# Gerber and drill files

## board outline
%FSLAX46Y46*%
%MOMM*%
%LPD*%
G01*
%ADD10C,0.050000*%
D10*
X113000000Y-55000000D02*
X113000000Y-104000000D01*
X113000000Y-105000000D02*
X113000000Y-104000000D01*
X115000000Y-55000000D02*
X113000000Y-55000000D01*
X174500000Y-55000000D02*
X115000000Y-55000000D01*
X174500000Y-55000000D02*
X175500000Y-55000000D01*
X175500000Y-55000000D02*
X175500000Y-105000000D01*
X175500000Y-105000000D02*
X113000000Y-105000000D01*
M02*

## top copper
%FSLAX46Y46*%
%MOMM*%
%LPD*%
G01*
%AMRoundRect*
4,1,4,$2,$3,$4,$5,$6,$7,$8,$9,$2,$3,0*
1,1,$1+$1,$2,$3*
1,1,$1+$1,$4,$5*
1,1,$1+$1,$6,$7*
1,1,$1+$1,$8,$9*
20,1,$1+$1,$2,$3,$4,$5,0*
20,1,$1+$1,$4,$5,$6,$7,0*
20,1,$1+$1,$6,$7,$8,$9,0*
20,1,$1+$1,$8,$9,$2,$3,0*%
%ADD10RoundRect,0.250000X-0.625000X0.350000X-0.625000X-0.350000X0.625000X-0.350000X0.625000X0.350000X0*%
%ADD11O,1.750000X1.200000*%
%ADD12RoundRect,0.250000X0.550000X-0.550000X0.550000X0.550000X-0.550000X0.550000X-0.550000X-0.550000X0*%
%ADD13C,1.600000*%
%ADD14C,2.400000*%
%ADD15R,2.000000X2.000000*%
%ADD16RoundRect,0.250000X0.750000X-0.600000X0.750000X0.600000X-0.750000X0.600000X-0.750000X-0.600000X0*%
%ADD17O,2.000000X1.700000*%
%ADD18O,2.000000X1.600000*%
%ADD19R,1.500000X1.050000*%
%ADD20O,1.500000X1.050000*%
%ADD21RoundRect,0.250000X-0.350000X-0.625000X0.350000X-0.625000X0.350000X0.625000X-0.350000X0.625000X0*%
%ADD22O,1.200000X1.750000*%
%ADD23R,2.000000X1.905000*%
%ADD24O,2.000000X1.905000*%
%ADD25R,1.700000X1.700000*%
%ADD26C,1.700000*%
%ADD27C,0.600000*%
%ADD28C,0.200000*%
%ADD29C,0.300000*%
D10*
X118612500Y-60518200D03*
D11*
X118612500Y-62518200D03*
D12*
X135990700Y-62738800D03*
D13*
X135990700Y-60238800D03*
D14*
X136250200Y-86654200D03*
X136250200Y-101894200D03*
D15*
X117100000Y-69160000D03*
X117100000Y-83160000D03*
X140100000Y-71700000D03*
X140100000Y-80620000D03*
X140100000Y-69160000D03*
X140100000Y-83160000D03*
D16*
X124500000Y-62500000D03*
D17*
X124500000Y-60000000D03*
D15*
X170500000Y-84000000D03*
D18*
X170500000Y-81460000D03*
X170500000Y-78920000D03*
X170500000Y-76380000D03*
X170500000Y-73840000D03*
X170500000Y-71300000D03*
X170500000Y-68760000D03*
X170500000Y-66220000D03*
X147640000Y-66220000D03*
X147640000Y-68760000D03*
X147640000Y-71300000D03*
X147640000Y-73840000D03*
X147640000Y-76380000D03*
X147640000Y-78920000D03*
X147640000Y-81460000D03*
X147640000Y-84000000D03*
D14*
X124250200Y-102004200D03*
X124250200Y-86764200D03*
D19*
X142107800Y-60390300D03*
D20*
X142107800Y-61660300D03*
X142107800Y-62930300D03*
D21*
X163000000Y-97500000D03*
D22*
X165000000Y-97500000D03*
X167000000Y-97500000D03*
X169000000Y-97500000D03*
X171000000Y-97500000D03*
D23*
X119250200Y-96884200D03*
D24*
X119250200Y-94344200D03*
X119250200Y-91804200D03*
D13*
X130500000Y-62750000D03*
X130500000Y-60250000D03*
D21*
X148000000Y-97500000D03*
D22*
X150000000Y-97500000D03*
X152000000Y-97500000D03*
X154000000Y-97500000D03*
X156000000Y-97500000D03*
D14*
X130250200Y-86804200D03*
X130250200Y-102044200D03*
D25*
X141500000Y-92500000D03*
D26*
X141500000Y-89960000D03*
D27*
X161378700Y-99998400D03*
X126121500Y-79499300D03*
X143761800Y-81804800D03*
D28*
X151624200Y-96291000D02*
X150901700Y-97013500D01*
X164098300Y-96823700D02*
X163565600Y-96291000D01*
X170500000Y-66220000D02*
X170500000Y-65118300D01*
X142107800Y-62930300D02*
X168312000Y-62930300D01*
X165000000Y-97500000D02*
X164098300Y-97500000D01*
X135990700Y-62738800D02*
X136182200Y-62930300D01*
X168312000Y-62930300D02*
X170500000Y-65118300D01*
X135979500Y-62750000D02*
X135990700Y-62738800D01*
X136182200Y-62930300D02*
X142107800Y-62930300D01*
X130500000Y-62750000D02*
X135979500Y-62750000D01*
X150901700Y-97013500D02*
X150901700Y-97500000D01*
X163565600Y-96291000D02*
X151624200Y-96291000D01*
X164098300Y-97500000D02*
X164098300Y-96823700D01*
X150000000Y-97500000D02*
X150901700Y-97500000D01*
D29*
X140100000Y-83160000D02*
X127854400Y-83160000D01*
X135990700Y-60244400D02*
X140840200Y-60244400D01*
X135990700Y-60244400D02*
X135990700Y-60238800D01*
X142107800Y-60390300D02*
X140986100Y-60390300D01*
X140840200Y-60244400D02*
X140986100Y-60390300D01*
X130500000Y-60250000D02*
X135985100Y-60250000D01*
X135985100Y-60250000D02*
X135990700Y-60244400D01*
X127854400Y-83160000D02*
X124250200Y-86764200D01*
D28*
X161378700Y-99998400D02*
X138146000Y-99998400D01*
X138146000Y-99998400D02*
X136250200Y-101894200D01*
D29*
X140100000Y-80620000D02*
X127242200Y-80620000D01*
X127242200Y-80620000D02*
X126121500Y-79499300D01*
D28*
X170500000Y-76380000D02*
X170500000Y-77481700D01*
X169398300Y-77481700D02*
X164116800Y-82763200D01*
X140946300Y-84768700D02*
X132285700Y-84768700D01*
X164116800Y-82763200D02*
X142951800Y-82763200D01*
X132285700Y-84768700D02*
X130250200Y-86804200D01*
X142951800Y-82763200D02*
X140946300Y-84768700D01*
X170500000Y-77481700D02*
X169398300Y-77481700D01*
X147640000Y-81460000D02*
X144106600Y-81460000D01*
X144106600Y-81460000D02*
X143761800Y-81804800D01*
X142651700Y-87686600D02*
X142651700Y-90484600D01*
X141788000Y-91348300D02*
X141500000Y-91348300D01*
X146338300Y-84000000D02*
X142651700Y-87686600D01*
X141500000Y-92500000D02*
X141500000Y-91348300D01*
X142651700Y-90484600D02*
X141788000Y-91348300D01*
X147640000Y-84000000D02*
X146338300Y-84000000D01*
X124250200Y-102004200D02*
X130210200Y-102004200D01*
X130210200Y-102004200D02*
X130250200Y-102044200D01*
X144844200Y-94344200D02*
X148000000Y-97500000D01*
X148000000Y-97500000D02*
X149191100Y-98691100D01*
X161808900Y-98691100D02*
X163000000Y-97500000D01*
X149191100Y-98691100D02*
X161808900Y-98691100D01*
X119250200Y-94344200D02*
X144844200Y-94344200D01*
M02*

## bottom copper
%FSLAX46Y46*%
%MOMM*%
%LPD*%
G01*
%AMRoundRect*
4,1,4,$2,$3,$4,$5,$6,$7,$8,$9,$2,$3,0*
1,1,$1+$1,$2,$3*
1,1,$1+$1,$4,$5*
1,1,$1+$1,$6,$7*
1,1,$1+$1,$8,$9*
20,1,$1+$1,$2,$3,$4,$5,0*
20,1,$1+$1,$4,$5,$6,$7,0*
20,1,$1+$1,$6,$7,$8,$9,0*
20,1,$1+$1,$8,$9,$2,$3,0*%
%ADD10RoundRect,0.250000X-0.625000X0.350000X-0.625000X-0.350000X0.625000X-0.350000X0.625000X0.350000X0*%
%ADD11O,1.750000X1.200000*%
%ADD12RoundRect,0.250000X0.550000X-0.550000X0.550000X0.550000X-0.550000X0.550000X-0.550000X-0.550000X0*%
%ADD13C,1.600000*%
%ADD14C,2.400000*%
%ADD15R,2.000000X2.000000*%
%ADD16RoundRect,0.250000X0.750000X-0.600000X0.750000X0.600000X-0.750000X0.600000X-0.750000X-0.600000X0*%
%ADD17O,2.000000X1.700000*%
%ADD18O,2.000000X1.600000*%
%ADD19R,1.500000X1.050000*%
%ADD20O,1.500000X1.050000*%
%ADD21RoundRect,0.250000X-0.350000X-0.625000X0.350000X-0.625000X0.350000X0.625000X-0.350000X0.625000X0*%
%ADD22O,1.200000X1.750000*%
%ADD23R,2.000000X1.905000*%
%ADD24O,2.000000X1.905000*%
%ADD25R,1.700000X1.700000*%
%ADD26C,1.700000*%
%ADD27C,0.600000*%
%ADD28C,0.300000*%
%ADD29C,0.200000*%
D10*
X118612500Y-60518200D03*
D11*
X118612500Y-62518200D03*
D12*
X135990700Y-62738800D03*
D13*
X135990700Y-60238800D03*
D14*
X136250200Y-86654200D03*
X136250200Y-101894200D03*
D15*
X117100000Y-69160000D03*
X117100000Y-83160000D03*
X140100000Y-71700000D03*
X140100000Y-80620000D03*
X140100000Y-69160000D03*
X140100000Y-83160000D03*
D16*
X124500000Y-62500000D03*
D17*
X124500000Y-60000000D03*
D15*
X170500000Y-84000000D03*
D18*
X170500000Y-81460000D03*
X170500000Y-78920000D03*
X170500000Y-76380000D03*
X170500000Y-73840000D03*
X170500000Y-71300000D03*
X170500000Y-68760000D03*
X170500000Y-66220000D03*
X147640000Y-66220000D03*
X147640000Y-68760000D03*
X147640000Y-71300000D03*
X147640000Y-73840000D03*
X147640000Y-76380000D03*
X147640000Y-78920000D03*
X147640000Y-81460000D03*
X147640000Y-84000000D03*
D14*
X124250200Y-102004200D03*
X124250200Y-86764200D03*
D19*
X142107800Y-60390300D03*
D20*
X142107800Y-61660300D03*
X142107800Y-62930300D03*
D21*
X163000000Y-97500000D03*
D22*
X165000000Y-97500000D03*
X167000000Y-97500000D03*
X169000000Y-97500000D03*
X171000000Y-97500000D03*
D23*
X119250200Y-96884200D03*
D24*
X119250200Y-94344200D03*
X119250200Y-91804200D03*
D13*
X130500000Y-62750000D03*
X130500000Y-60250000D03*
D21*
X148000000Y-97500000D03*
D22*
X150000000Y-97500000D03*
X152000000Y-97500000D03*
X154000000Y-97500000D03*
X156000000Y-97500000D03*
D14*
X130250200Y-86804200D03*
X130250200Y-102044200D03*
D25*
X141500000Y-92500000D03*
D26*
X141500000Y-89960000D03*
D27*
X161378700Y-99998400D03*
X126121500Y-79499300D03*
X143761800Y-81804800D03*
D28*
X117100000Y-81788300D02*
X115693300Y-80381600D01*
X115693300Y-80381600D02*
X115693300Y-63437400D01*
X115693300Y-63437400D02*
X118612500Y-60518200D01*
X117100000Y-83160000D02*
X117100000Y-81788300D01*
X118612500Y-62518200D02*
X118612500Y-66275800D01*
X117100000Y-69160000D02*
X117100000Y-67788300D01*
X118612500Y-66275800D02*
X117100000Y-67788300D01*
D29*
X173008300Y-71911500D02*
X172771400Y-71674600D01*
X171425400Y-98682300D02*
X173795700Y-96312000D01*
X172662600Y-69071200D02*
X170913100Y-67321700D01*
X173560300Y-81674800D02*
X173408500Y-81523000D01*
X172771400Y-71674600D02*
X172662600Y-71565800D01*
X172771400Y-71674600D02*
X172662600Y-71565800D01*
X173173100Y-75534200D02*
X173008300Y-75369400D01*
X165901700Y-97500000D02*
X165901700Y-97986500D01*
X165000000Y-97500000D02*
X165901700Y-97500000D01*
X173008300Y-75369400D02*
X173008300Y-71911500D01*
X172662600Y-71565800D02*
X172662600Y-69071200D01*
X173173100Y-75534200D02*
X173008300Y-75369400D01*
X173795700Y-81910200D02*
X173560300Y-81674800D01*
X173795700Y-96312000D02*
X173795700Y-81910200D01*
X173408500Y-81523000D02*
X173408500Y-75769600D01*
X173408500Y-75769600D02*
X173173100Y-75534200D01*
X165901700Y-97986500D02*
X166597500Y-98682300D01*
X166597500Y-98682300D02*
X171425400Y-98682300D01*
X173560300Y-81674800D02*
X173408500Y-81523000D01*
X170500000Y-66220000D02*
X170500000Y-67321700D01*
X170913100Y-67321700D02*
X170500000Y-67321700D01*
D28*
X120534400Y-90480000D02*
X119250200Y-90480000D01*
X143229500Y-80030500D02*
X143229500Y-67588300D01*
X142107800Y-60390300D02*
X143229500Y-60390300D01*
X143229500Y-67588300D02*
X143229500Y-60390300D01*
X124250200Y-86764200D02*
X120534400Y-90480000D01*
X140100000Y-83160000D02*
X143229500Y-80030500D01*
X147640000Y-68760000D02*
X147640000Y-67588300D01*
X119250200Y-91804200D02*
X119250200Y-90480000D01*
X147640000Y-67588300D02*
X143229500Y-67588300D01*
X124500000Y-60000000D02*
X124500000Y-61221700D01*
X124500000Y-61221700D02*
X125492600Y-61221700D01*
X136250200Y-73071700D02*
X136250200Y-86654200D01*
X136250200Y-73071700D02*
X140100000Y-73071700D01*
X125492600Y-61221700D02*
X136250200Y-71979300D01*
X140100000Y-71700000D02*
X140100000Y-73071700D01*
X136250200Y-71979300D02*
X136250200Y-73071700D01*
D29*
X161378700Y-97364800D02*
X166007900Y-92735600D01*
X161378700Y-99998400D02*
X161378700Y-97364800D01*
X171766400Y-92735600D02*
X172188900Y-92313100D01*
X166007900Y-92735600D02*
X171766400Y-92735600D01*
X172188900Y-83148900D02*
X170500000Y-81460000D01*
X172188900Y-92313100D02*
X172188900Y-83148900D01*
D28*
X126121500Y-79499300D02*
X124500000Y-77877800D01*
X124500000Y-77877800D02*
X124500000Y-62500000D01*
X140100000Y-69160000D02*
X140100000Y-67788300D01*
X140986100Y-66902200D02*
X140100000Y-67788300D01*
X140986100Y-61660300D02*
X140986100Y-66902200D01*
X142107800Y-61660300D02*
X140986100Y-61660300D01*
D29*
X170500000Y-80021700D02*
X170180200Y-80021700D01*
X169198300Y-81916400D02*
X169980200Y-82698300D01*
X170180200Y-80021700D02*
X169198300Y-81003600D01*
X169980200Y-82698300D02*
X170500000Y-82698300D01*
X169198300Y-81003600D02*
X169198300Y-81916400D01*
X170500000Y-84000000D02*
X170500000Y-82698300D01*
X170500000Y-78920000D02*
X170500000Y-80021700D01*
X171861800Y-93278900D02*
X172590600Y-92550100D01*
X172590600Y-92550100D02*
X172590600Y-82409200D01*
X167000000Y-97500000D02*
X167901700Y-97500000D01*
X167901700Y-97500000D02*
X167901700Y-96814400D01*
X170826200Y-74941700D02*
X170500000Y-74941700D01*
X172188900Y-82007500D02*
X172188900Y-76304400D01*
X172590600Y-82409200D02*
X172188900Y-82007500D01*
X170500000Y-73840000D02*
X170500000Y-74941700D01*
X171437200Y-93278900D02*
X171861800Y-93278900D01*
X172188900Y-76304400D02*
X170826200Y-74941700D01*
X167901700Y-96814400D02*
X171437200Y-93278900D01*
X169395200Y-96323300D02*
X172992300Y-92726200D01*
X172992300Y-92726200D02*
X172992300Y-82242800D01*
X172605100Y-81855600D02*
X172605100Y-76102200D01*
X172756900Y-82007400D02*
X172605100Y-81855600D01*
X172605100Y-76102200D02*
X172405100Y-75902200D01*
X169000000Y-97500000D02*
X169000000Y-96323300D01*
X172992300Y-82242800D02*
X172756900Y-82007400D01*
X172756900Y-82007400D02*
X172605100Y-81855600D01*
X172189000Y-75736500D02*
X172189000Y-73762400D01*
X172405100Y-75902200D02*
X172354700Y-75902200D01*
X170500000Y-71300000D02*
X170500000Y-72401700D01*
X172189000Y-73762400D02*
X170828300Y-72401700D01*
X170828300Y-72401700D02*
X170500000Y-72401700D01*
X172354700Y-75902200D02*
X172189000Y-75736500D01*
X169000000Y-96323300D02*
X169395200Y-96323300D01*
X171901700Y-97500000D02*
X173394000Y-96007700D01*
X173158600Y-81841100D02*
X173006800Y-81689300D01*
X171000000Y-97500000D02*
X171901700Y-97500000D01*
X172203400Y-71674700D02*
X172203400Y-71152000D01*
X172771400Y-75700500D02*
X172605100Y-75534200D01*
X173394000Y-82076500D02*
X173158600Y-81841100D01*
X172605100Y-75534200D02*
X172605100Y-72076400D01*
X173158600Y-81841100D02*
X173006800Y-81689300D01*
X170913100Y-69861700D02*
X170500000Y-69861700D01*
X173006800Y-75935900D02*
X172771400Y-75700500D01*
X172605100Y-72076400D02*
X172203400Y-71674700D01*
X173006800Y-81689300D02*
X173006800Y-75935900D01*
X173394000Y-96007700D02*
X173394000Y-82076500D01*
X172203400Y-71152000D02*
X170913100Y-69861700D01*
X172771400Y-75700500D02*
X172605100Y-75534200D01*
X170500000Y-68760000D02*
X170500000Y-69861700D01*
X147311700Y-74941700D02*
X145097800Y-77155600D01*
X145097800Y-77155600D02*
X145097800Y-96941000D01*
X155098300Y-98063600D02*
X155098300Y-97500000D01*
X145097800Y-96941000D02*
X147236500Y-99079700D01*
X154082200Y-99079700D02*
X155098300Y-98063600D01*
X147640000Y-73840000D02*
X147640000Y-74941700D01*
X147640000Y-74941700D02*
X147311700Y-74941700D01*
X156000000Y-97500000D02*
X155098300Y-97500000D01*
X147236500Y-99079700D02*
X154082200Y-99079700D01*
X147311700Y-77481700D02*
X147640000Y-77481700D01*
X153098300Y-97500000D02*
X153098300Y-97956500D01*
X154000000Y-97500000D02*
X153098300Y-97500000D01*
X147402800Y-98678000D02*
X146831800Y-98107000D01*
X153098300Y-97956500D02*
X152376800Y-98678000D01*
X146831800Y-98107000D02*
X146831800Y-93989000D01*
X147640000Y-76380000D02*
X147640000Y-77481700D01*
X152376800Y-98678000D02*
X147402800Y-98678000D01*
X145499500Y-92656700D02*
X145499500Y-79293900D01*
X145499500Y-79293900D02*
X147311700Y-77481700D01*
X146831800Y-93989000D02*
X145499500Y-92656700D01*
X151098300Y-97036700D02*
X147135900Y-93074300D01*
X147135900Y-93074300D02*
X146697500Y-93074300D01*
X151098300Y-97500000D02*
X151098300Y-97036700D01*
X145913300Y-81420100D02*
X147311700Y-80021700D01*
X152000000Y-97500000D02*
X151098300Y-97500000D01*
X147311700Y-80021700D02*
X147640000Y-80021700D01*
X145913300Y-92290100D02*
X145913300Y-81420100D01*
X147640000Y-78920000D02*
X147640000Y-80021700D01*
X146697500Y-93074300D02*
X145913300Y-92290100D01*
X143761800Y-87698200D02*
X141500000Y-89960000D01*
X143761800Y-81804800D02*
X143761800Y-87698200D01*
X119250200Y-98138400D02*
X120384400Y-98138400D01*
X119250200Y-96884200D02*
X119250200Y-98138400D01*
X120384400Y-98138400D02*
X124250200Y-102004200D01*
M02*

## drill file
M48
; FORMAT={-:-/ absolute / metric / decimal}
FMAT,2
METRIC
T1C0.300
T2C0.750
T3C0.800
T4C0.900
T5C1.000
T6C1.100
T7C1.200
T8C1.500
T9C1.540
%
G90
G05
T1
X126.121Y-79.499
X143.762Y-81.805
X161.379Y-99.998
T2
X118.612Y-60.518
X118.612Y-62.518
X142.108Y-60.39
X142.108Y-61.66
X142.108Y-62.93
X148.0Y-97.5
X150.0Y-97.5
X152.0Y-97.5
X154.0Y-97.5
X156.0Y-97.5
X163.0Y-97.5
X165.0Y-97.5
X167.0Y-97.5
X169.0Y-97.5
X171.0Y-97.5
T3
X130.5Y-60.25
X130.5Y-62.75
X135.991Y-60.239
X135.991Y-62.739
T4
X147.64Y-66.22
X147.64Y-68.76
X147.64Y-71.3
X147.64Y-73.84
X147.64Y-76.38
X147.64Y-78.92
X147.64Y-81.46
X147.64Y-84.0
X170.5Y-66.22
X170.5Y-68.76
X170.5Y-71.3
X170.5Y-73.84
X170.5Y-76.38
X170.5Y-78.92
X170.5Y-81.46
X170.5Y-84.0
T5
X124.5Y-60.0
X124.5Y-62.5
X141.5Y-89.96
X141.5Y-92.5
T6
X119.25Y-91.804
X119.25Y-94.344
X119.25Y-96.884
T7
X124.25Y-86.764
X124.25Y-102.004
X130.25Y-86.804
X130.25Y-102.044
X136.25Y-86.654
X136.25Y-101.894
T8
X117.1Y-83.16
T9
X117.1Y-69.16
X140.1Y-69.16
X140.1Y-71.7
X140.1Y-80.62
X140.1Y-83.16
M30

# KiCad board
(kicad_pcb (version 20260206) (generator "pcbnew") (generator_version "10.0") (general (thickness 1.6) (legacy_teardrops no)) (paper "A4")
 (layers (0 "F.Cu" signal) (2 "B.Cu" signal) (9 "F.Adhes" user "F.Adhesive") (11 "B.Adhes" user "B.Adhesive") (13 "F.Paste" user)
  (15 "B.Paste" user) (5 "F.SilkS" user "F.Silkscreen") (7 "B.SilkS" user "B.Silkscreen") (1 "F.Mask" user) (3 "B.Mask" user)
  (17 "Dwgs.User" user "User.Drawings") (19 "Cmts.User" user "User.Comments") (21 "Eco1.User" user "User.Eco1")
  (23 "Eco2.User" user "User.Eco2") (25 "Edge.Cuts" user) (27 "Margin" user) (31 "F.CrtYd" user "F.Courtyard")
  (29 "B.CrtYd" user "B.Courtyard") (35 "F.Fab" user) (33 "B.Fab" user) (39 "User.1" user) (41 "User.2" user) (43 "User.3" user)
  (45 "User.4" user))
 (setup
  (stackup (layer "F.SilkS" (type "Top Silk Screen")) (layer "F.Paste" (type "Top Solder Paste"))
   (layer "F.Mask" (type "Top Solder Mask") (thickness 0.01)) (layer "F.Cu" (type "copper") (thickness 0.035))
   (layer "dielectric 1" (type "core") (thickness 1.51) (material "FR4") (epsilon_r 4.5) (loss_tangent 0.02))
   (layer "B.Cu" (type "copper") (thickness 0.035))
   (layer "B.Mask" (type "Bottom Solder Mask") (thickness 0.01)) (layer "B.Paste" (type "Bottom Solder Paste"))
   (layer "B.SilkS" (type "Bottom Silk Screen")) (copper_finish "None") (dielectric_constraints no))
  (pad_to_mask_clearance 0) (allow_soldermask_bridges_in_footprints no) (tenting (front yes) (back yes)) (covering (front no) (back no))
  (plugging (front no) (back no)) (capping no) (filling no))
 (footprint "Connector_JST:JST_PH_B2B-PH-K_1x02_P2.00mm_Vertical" (layer "F.Cu") (at 118.6125 60.5182 -90)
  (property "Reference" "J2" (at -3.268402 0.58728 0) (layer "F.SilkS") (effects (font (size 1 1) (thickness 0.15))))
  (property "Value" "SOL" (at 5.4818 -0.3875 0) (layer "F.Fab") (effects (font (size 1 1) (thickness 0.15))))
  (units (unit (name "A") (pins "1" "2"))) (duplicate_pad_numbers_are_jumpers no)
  (pad "1" thru_hole roundrect (at 0 0 270) (size 1.2 1.75) (drill 0.75) (layers "*.Cu" "*.Mask") (remove_unused_layers no)
   (roundrect_rratio 0.208333) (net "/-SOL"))
  (pad "2" thru_hole oval (at 2 0 270) (size 1.2 1.75) (drill 0.75) (layers "*.Cu" "*.Mask") (remove_unused_layers no) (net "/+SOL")))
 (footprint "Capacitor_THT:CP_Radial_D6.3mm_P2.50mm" (layer "F.Cu") (at 135.9907 62.7388 90)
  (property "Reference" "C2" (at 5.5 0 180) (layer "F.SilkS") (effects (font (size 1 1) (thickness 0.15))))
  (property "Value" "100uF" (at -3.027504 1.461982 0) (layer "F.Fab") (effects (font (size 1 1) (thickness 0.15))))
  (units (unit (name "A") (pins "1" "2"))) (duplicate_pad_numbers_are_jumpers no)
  (pad "1" thru_hole roundrect (at 0 0 90) (size 1.6 1.6) (drill 0.8) (layers "*.Cu" "*.Mask") (remove_unused_layers no)
   (roundrect_rratio 0.15625) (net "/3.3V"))
  (pad "2" thru_hole circle (at 2.5 0 90) (size 1.6 1.6) (drill 0.8) (layers "*.Cu" "*.Mask") (remove_unused_layers no) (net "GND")))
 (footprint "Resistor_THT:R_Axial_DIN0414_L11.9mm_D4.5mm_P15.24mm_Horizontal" (layer "F.Cu") (at 136.2502 86.6542 -90)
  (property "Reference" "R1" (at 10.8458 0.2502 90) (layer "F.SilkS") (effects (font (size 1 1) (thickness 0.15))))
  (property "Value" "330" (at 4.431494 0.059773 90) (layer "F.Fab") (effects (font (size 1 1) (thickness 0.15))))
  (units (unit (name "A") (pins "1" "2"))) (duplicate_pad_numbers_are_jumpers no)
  (pad "1" thru_hole circle (at 0 0 270) (size 2.4 2.4) (drill 1.2) (layers "*.Cu" "*.Mask") (remove_unused_layers no) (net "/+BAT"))
  (pad "2" thru_hole circle (at 15.24 0 270) (size 2.4 2.4) (drill 1.2) (layers "*.Cu" "*.Mask") (remove_unused_layers no)
   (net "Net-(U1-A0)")))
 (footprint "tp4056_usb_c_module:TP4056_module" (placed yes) (layer "F.Cu") (at 115.5 67.5)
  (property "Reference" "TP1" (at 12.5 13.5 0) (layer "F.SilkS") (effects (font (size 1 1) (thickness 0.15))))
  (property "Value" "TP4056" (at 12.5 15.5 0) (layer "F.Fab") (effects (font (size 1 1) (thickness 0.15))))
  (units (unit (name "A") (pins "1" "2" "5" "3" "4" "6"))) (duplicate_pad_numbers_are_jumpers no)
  (pad "1" thru_hole rect (at 1.6 1.66) (size 2 2) (drill 1.54) (layers "*.Cu" "*.Mask") (remove_unused_layers no) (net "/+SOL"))
  (pad "2" thru_hole rect (at 1.6 15.66) (size 2 2) (drill 1.5) (layers "*.Cu" "*.Mask") (remove_unused_layers no) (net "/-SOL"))
  (pad "3" thru_hole rect (at 24.6 4.2) (size 2 2) (drill 1.54) (layers "*.Cu" "*.Mask") (remove_unused_layers no) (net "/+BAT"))
  (pad "4" thru_hole rect (at 24.6 13.12) (size 2 2) (drill 1.54) (layers "*.Cu" "*.Mask") (remove_unused_layers no) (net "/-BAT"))
  (pad "5" thru_hole rect (at 24.6 1.66) (size 2 2) (drill 1.54) (layers "*.Cu" "*.Mask") (remove_unused_layers no) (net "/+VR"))
  (pad "6" thru_hole rect (at 24.6 15.66) (size 2 2) (drill 1.54) (layers "*.Cu" "*.Mask") (remove_unused_layers no) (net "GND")))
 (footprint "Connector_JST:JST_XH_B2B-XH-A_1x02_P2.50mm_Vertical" (layer "F.Cu") (at 124.5 62.5 90)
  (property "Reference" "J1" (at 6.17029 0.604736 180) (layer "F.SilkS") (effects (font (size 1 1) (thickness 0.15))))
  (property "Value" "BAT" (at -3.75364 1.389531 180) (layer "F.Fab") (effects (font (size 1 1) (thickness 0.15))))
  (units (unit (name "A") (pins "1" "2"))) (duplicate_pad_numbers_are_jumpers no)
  (pad "1" thru_hole roundrect (at 0 0 90) (size 1.7 2) (drill 1) (layers "*.Cu" "*.Mask") (remove_unused_layers no)
   (roundrect_rratio 0.147059) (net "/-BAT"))
  (pad "2" thru_hole oval (at 2.5 0 90) (size 1.7 2) (drill 1) (layers "*.Cu" "*.Mask") (remove_unused_layers no) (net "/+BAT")))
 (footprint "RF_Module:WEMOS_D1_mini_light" (layer "F.Cu") (at 170.5 84 180)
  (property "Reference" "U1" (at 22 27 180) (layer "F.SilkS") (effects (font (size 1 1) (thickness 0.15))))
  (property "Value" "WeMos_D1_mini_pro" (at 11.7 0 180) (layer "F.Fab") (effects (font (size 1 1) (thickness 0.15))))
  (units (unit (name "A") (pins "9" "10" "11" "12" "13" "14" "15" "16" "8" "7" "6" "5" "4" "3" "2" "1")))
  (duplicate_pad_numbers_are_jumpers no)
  (pad "1" thru_hole rect (at 0 0 180) (size 2 2) (drill 0.9) (layers "*.Cu" "*.Mask") (remove_unused_layers no) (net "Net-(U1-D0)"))
  (pad "2" thru_hole oval (at 0 2.54 180) (size 2 1.6) (drill 0.9) (layers "*.Cu" "*.Mask") (remove_unused_layers no) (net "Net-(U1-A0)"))
  (pad "3" thru_hole oval (at 0 5.08 180) (size 2 1.6) (drill 0.9) (layers "*.Cu" "*.Mask") (remove_unused_layers no) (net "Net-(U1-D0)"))
  (pad "4" thru_hole oval (at 0 7.62 180) (size 2 1.6) (drill 0.9) (layers "*.Cu" "*.Mask") (remove_unused_layers no) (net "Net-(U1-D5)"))
  (pad "5" thru_hole oval (at 0 10.16 180) (size 2 1.6) (drill 0.9) (layers "*.Cu" "*.Mask") (remove_unused_layers no) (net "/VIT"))
  (pad "6" thru_hole oval (at 0 12.7 180) (size 2 1.6) (drill 0.9) (layers "*.Cu" "*.Mask") (remove_unused_layers no) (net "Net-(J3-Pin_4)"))
  (pad "7" thru_hole oval (at 0 15.24 180) (size 2 1.6) (drill 0.9) (layers "*.Cu" "*.Mask") (remove_unused_layers no)
   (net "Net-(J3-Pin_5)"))
  (pad "8" thru_hole oval (at 0 17.78 180) (size 2 1.6) (drill 0.9) (layers "*.Cu" "*.Mask") (remove_unused_layers no) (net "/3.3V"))
  (pad "9" thru_hole oval (at 22.86 17.78 180) (size 2 1.6) (drill 0.9) (layers "*.Cu" "*.Mask") (remove_unused_layers no)
   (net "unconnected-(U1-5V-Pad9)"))
  (pad "10" thru_hole oval (at 22.86 15.24 180) (size 2 1.6) (drill 0.9) (layers "*.Cu" "*.Mask") (remove_unused_layers no) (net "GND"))
  (pad "11" thru_hole oval (at 22.86 12.7 180) (size 2 1.6) (drill 0.9) (layers "*.Cu" "*.Mask") (remove_unused_layers no)
   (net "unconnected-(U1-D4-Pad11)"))
  (pad "12" thru_hole oval (at 22.86 10.16 180) (size 2 1.6) (drill 0.9) (layers "*.Cu" "*.Mask") (remove_unused_layers no)
   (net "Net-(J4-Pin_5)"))
  (pad "13" thru_hole oval (at 22.86 7.62 180) (size 2 1.6) (drill 0.9) (layers "*.Cu" "*.Mask") (remove_unused_layers no)
   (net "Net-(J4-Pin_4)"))
  (pad "14" thru_hole oval (at 22.86 5.08 180) (size 2 1.6) (drill 0.9) (layers "*.Cu" "*.Mask") (remove_unused_layers no)
   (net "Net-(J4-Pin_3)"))
  (pad "15" thru_hole oval (at 22.86 2.54 180) (size 2 1.6) (drill 0.9) (layers "*.Cu" "*.Mask") (remove_unused_layers no) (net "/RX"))
  (pad "16" thru_hole oval (at 22.86 0 180) (size 2 1.6) (drill 0.9) (layers "*.Cu" "*.Mask") (remove_unused_layers no) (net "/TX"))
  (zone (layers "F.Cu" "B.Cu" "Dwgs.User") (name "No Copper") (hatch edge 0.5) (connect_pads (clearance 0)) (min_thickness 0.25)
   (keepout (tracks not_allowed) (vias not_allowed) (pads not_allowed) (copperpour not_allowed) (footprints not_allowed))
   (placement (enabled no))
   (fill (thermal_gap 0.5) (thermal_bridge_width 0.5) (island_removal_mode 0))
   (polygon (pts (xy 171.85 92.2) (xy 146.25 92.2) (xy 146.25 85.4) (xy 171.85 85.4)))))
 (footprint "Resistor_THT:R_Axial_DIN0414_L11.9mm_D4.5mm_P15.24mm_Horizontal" (layer "F.Cu") (at 124.2502 102.0042 90)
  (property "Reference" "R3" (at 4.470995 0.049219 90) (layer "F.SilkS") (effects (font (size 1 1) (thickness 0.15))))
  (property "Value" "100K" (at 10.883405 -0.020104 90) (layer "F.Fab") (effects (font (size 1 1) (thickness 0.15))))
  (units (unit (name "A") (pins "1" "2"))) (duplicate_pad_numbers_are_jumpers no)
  (pad "1" thru_hole circle (at 0 0 90) (size 2.4 2.4) (drill 1.2) (layers "*.Cu" "*.Mask") (remove_unused_layers no) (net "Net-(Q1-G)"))
  (pad "2" thru_hole circle (at 15.24 0 90) (size 2.4 2.4) (drill 1.2) (layers "*.Cu" "*.Mask") (remove_unused_layers no) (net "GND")))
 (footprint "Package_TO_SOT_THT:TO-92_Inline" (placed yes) (layer "F.Cu") (at 142.1078 60.3903 -90)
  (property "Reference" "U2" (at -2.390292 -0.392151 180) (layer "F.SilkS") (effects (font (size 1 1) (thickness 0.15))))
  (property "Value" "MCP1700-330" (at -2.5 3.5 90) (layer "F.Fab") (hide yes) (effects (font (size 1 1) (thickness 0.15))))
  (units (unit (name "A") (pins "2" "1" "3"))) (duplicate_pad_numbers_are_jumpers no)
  (pad "1" thru_hole rect (at 0 0 270) (size 1.05 1.5) (drill 0.75) (layers "*.Cu" "*.Mask") (remove_unused_layers no) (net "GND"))
  (pad "2" thru_hole oval (at 1.27 0 270) (size 1.05 1.5) (drill 0.75) (layers "*.Cu" "*.Mask") (remove_unused_layers no) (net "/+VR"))
  (pad "3" thru_hole oval (at 2.54 0 270) (size 1.05 1.5) (drill 0.75) (layers "*.Cu" "*.Mask") (remove_unused_layers no) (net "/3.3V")))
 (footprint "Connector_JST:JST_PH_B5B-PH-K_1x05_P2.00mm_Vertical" (layer "F.Cu") (at 163 97.5)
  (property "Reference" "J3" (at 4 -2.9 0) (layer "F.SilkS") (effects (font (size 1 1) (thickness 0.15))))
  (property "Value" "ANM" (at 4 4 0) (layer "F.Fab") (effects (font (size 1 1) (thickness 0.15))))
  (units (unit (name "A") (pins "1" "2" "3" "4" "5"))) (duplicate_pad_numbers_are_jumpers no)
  (pad "1" thru_hole roundrect (at 0 0) (size 1.2 1.75) (drill 0.75) (layers "*.Cu" "*.Mask") (remove_unused_layers no)
   (roundrect_rratio 0.208333) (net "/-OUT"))
  (pad "2" thru_hole oval (at 2 0) (size 1.2 1.75) (drill 0.75) (layers "*.Cu" "*.Mask") (remove_unused_layers no) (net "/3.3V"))
  (pad "3" thru_hole oval (at 4 0) (size 1.2 1.75) (drill 0.75) (layers "*.Cu" "*.Mask") (remove_unused_layers no) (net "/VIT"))
  (pad "4" thru_hole oval (at 6 0) (size 1.2 1.75) (drill 0.75) (layers "*.Cu" "*.Mask") (remove_unused_layers no) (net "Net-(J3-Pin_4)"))
  (pad "5" thru_hole oval (at 8 0) (size 1.2 1.75) (drill 0.75) (layers "*.Cu" "*.Mask") (remove_unused_layers no) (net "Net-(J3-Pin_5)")))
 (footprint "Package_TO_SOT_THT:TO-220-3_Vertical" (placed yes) (layer "F.Cu") (at 119.2502 96.8842 90)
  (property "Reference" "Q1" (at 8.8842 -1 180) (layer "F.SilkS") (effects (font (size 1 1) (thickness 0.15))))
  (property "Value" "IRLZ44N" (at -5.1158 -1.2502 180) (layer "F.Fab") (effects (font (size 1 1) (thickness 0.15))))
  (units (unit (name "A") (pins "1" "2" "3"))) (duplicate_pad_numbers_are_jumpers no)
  (pad "1" thru_hole rect (at 0 0 90) (size 1.905 2) (drill 1.1) (layers "*.Cu" "*.Mask") (remove_unused_layers no) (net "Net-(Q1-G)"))
  (pad "2" thru_hole oval (at 2.54 0 90) (size 1.905 2) (drill 1.1) (layers "*.Cu" "*.Mask") (remove_unused_layers no) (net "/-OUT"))
  (pad "3" thru_hole oval (at 5.08 0 90) (size 1.905 2) (drill 1.1) (layers "*.Cu" "*.Mask") (remove_unused_layers no) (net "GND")))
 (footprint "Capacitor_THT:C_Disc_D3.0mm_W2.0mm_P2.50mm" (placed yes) (layer "F.Cu") (at 130.5 62.75 90)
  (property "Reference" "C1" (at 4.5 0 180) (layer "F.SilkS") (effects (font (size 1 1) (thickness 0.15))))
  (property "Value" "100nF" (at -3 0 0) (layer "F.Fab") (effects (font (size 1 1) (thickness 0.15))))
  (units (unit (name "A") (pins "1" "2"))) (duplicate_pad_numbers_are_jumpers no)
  (pad "1" thru_hole circle (at 0 0 90) (size 1.6 1.6) (drill 0.8) (layers "*.Cu" "*.Mask") (remove_unused_layers no) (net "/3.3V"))
  (pad "2" thru_hole circle (at 2.5 0 90) (size 1.6 1.6) (drill 0.8) (layers "*.Cu" "*.Mask") (remove_unused_layers no) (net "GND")))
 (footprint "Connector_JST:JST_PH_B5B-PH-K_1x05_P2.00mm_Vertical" (layer "F.Cu") (at 148 97.5)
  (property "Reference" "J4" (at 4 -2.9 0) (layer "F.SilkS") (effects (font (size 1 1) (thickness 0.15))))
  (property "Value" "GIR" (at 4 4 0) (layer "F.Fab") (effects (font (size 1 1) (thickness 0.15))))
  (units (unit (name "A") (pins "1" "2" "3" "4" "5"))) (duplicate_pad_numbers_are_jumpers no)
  (pad "1" thru_hole roundrect (at 0 0) (size 1.2 1.75) (drill 0.75) (layers "*.Cu" "*.Mask") (remove_unused_layers no)
   (roundrect_rratio 0.208333) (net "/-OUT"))
  (pad "2" thru_hole oval (at 2 0) (size 1.2 1.75) (drill 0.75) (layers "*.Cu" "*.Mask") (remove_unused_layers no) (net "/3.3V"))
  (pad "3" thru_hole oval (at 4 0) (size 1.2 1.75) (drill 0.75) (layers "*.Cu" "*.Mask") (remove_unused_layers no) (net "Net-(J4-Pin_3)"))
  (pad "4" thru_hole oval (at 6 0) (size 1.2 1.75) (drill 0.75) (layers "*.Cu" "*.Mask") (remove_unused_layers no) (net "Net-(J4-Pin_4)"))
  (pad "5" thru_hole oval (at 8 0) (size 1.2 1.75) (drill 0.75) (layers "*.Cu" "*.Mask") (remove_unused_layers no) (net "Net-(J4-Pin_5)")))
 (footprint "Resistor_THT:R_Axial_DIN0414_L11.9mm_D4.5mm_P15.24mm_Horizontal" (layer "F.Cu") (at 130.2502 86.8042 -90)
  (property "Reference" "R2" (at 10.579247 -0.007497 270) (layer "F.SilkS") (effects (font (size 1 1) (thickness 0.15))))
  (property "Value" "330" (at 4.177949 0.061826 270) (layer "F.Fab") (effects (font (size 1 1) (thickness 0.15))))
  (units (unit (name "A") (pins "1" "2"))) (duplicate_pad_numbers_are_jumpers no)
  (pad "1" thru_hole circle (at 0 0 270) (size 2.4 2.4) (drill 1.2) (layers "*.Cu" "*.Mask") (remove_unused_layers no) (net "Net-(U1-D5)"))
  (pad "2" thru_hole circle (at 15.24 0 270) (size 2.4 2.4) (drill 1.2) (layers "*.Cu" "*.Mask") (remove_unused_layers no)
   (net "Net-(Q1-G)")))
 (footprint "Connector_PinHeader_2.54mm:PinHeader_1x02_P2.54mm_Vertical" (layer "F.Cu") (at 141.5 92.5 180)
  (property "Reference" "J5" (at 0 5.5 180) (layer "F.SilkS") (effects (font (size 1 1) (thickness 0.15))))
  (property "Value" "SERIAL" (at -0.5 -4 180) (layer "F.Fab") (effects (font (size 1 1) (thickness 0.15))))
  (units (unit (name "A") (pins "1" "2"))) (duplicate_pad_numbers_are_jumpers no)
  (pad "1" thru_hole rect (at 0 0 180) (size 1.7 1.7) (drill 1) (layers "*.Cu" "*.Mask") (remove_unused_layers no) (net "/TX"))
  (pad "2" thru_hole circle (at 0 2.54 180) (size 1.7 1.7) (drill 1) (layers "*.Cu" "*.Mask") (remove_unused_layers no) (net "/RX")))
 (gr_line (start 113 55) (end 113 104) (stroke (width 0.05) (type default)) (layer "Edge.Cuts"))
 (gr_line (start 113 105) (end 113 104) (stroke (width 0.05) (type default)) (layer "Edge.Cuts"))
 (gr_line (start 115 55) (end 113 55) (stroke (width 0.05) (type default)) (layer "Edge.Cuts"))
 (gr_line (start 174.5 55) (end 115 55) (stroke (width 0.05) (type default)) (layer "Edge.Cuts"))
 (gr_line (start 174.5 55) (end 175.5 55) (stroke (width 0.05) (type default)) (layer "Edge.Cuts"))
 (gr_line (start 175.5 55) (end 175.5 105) (stroke (width 0.05) (type default)) (layer "Edge.Cuts"))
 (gr_line (start 175.5 105) (end 113 105) (stroke (width 0.05) (type default)) (layer "Edge.Cuts"))
 (segment (start 117.1 81.7883) (end 115.6933 80.3816) (width 0.3) (layer "B.Cu") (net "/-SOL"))
 (segment (start 115.6933 80.3816) (end 115.6933 63.4374) (width 0.3) (layer "B.Cu") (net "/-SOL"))
 (segment (start 115.6933 63.4374) (end 118.6125 60.5182) (width 0.3) (layer "B.Cu") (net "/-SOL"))
 (segment (start 117.1 83.16) (end 117.1 81.7883) (width 0.3) (layer "B.Cu") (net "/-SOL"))
 (segment (start 118.6125 62.5182) (end 118.6125 66.2758) (width 0.3) (layer "B.Cu") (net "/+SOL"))
 (segment (start 117.1 69.16) (end 117.1 67.7883) (width 0.3) (layer "B.Cu") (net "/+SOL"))
 (segment (start 118.6125 66.2758) (end 117.1 67.7883) (width 0.3) (layer "B.Cu") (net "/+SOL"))
 (segment (start 151.6242 96.291) (end 150.9017 97.0135) (width 0.2) (layer "F.Cu") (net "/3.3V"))
 (segment (start 164.0983 96.8237) (end 163.5656 96.291) (width 0.2) (layer "F.Cu") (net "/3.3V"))
 (segment (start 170.5 66.22) (end 170.5 65.1183) (width 0.2) (layer "F.Cu") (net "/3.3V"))
 (segment (start 142.1078 62.9303) (end 168.312 62.9303) (width 0.2) (layer "F.Cu") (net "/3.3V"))
 (segment (start 165 97.5) (end 164.0983 97.5) (width 0.2) (layer "F.Cu") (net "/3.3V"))
 (segment (start 135.9907 62.7388) (end 136.1822 62.9303) (width 0.2) (layer "F.Cu") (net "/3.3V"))
 (segment (start 168.312 62.9303) (end 170.5 65.1183) (width 0.2) (layer "F.Cu") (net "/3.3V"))
 (segment (start 135.9795 62.75) (end 135.9907 62.7388) (width 0.2) (layer "F.Cu") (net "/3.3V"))
 (segment (start 136.1822 62.9303) (end 142.1078 62.9303) (width 0.2) (layer "F.Cu") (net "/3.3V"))
 (segment (start 130.5 62.75) (end 135.9795 62.75) (width 0.2) (layer "F.Cu") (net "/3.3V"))
 (segment (start 150.9017 97.0135) (end 150.9017 97.5) (width 0.2) (layer "F.Cu") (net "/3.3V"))
 (segment (start 163.5656 96.291) (end 151.6242 96.291) (width 0.2) (layer "F.Cu") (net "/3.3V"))
 (segment (start 164.0983 97.5) (end 164.0983 96.8237) (width 0.2) (layer "F.Cu") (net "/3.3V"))
 (segment (start 150 97.5) (end 150.9017 97.5) (width 0.2) (layer "F.Cu") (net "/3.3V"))
 (segment (start 173.0083 71.9115) (end 172.7714 71.6746) (width 0.2) (layer "B.Cu") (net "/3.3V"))
 (segment (start 171.4254 98.6823) (end 173.7957 96.312) (width 0.2) (layer "B.Cu") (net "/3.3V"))
 (segment (start 172.6626 69.0712) (end 170.9131 67.3217) (width 0.2) (layer "B.Cu") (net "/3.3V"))
 (segment (start 173.5603 81.6748) (end 173.4085 81.523) (width 0.2) (layer "B.Cu") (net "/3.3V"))
 (segment (start 172.7714 71.6746) (end 172.6626 71.5658) (width 0.2) (layer "B.Cu") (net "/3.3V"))
 (segment (start 172.7714 71.6746) (end 172.6626 71.5658) (width 0.2) (layer "B.Cu") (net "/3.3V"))
 (segment (start 173.1731 75.5342) (end 173.0083 75.3694) (width 0.2) (layer "B.Cu") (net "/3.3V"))
 (segment (start 165.9017 97.5) (end 165.9017 97.9865) (width 0.2) (layer "B.Cu") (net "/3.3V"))
 (segment (start 165 97.5) (end 165.9017 97.5) (width 0.2) (layer "B.Cu") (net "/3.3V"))
 (segment (start 173.0083 75.3694) (end 173.0083 71.9115) (width 0.2) (layer "B.Cu") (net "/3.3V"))
 (segment (start 172.6626 71.5658) (end 172.6626 69.0712) (width 0.2) (layer "B.Cu") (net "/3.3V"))
 (segment (start 173.1731 75.5342) (end 173.0083 75.3694) (width 0.2) (layer "B.Cu") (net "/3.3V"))
 (segment (start 173.7957 81.9102) (end 173.5603 81.6748) (width 0.2) (layer "B.Cu") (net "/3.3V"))
 (segment (start 173.7957 96.312) (end 173.7957 81.9102) (width 0.2) (layer "B.Cu") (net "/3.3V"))
 (segment (start 173.4085 81.523) (end 173.4085 75.7696) (width 0.2) (layer "B.Cu") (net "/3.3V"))
 (segment (start 173.4085 75.7696) (end 173.1731 75.5342) (width 0.2) (layer "B.Cu") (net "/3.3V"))
 (segment (start 165.9017 97.9865) (end 166.5975 98.6823) (width 0.2) (layer "B.Cu") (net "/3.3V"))
 (segment (start 166.5975 98.6823) (end 171.4254 98.6823) (width 0.2) (layer "B.Cu") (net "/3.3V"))
 (segment (start 173.5603 81.6748) (end 173.4085 81.523) (width 0.2) (layer "B.Cu") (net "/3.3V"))
 (segment (start 170.5 66.22) (end 170.5 67.3217) (width 0.2) (layer "B.Cu") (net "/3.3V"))
 (segment (start 170.9131 67.3217) (end 170.5 67.3217) (width 0.2) (layer "B.Cu") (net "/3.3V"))
 (segment (start 140.1 83.16) (end 127.8544 83.16) (width 0.3) (layer "F.Cu") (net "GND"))
 (segment (start 135.9907 60.2444) (end 140.8402 60.2444) (width 0.3) (layer "F.Cu") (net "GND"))
 (segment (start 135.9907 60.2444) (end 135.9907 60.2388) (width 0.3) (layer "F.Cu") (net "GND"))
 (segment (start 142.1078 60.3903) (end 140.9861 60.3903) (width 0.3) (layer "F.Cu") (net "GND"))
 (segment (start 140.8402 60.2444) (end 140.9861 60.3903) (width 0.3) (layer "F.Cu") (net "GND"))
 (segment (start 130.5 60.25) (end 135.9851 60.25) (width 0.3) (layer "F.Cu") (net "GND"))
 (segment (start 135.9851 60.25) (end 135.9907 60.2444) (width 0.3) (layer "F.Cu") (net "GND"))
 (segment (start 127.8544 83.16) (end 124.2502 86.7642) (width 0.3) (layer "F.Cu") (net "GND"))
 (segment (start 120.5344 90.48) (end 119.2502 90.48) (width 0.3) (layer "B.Cu") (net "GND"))
 (segment (start 143.2295 80.0305) (end 143.2295 67.5883) (width 0.3) (layer "B.Cu") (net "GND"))
 (segment (start 142.1078 60.3903) (end 143.2295 60.3903) (width 0.3) (layer "B.Cu") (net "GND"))
 (segment (start 143.2295 67.5883) (end 143.2295 60.3903) (width 0.3) (layer "B.Cu") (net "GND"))
 (segment (start 124.2502 86.7642) (end 120.5344 90.48) (width 0.3) (layer "B.Cu") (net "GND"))
 (segment (start 140.1 83.16) (end 143.2295 80.0305) (width 0.3) (layer "B.Cu") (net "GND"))
 (segment (start 147.64 68.76) (end 147.64 67.5883) (width 0.3) (layer "B.Cu") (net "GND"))
 (segment (start 119.2502 91.8042) (end 119.2502 90.48) (width 0.3) (layer "B.Cu") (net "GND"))
 (segment (start 147.64 67.5883) (end 143.2295 67.5883) (width 0.3) (layer "B.Cu") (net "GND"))
 (segment (start 124.5 60) (end 124.5 61.2217) (width 0.3) (layer "B.Cu") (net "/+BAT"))
 (segment (start 124.5 61.2217) (end 125.4926 61.2217) (width 0.3) (layer "B.Cu") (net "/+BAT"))
 (segment (start 136.2502 73.0717) (end 136.2502 86.6542) (width 0.3) (layer "B.Cu") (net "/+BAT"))
 (segment (start 136.2502 73.0717) (end 140.1 73.0717) (width 0.3) (layer "B.Cu") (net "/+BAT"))
 (segment (start 125.4926 61.2217) (end 136.2502 71.9793) (width 0.3) (layer "B.Cu") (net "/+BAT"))
 (segment (start 140.1 71.7) (end 140.1 73.0717) (width 0.3) (layer "B.Cu") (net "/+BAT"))
 (segment (start 136.2502 71.9793) (end 136.2502 73.0717) (width 0.3) (layer "B.Cu") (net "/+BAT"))
 (segment (start 161.3787 99.9984) (end 138.146 99.9984) (width 0.2) (layer "F.Cu") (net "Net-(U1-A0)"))
 (segment (start 138.146 99.9984) (end 136.2502 101.8942) (width 0.2) (layer "F.Cu") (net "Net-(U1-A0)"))
 (via (at 161.3787 99.9984) (size 0.6) (drill 0.3) (layers "F.Cu" "B.Cu") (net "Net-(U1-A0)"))
 (segment (start 161.3787 97.3648) (end 166.0079 92.7356) (width 0.2) (layer "B.Cu") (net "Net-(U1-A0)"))
 (segment (start 161.3787 99.9984) (end 161.3787 97.3648) (width 0.2) (layer "B.Cu") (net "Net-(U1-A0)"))
 (segment (start 171.7664 92.7356) (end 172.1889 92.3131) (width 0.2) (layer "B.Cu") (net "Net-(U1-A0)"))
 (segment (start 166.0079 92.7356) (end 171.7664 92.7356) (width 0.2) (layer "B.Cu") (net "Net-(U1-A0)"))
 (segment (start 172.1889 83.1489) (end 170.5 81.46) (width 0.2) (layer "B.Cu") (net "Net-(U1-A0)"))
 (segment (start 172.1889 92.3131) (end 172.1889 83.1489) (width 0.2) (layer "B.Cu") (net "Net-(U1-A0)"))
 (segment (start 140.1 80.62) (end 127.2422 80.62) (width 0.3) (layer "F.Cu") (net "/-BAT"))
 (segment (start 127.2422 80.62) (end 126.1215 79.4993) (width 0.3) (layer "F.Cu") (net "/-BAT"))
 (via (at 126.1215 79.4993) (size 0.6) (drill 0.3) (layers "F.Cu" "B.Cu") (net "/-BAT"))
 (segment (start 126.1215 79.4993) (end 124.5 77.8778) (width 0.3) (layer "B.Cu") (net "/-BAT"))
 (segment (start 124.5 77.8778) (end 124.5 62.5) (width 0.3) (layer "B.Cu") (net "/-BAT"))
 (segment (start 140.1 69.16) (end 140.1 67.7883) (width 0.3) (layer "B.Cu") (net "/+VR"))
 (segment (start 140.9861 66.9022) (end 140.1 67.7883) (width 0.3) (layer "B.Cu") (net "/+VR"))
 (segment (start 140.9861 61.6603) (end 140.9861 66.9022) (width 0.3) (layer "B.Cu") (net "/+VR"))
 (segment (start 142.1078 61.6603) (end 140.9861 61.6603) (width 0.3) (layer "B.Cu") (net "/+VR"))
 (segment (start 170.5 80.0217) (end 170.1802 80.0217) (width 0.2) (layer "B.Cu") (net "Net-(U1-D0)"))
 (segment (start 169.1983 81.9164) (end 169.9802 82.6983) (width 0.2) (layer "B.Cu") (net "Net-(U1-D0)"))
 (segment (start 170.1802 80.0217) (end 169.1983 81.0036) (width 0.2) (layer "B.Cu") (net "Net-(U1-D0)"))
 (segment (start 169.9802 82.6983) (end 170.5 82.6983) (width 0.2) (layer "B.Cu") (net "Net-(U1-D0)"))
 (segment (start 169.1983 81.0036) (end 169.1983 81.9164) (width 0.2) (layer "B.Cu") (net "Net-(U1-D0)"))
 (segment (start 170.5 84) (end 170.5 82.6983) (width 0.2) (layer "B.Cu") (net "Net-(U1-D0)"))
 (segment (start 170.5 78.92) (end 170.5 80.0217) (width 0.2) (layer "B.Cu") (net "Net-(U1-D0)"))
 (segment (start 170.5 76.38) (end 170.5 77.4817) (width 0.2) (layer "F.Cu") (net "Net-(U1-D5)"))
 (segment (start 169.3983 77.4817) (end 164.1168 82.7632) (width 0.2) (layer "F.Cu") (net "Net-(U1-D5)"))
 (segment (start 140.9463 84.7687) (end 132.2857 84.7687) (width 0.2) (layer "F.Cu") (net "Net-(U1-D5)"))
 (segment (start 164.1168 82.7632) (end 142.9518 82.7632) (width 0.2) (layer "F.Cu") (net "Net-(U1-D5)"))
 (segment (start 132.2857 84.7687) (end 130.2502 86.8042) (width 0.2) (layer "F.Cu") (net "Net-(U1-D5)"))
 (segment (start 142.9518 82.7632) (end 140.9463 84.7687) (width 0.2) (layer "F.Cu") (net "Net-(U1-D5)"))
 (segment (start 170.5 77.4817) (end 169.3983 77.4817) (width 0.2) (layer "F.Cu") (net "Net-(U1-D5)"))
 (segment (start 171.8618 93.2789) (end 172.5906 92.5501) (width 0.2) (layer "B.Cu") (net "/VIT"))
 (segment (start 172.5906 92.5501) (end 172.5906 82.4092) (width 0.2) (layer "B.Cu") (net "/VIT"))
 (segment (start 167 97.5) (end 167.9017 97.5) (width 0.2) (layer "B.Cu") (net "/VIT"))
 (segment (start 167.9017 97.5) (end 167.9017 96.8144) (width 0.2) (layer "B.Cu") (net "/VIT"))
 (segment (start 170.8262 74.9417) (end 170.5 74.9417) (width 0.2) (layer "B.Cu") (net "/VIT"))
 (segment (start 172.1889 82.0075) (end 172.1889 76.3044) (width 0.2) (layer "B.Cu") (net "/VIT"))
 (segment (start 172.5906 82.4092) (end 172.1889 82.0075) (width 0.2) (layer "B.Cu") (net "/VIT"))
 (segment (start 170.5 73.84) (end 170.5 74.9417) (width 0.2) (layer "B.Cu") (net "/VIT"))
 (segment (start 171.4372 93.2789) (end 171.8618 93.2789) (width 0.2) (layer "B.Cu") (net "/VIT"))
 (segment (start 172.1889 76.3044) (end 170.8262 74.9417) (width 0.2) (layer "B.Cu") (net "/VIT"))
 (segment (start 167.9017 96.8144) (end 171.4372 93.2789) (width 0.2) (layer "B.Cu") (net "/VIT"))
 (segment (start 169.3952 96.3233) (end 172.9923 92.7262) (width 0.2) (layer "B.Cu") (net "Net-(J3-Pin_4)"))
 (segment (start 172.9923 92.7262) (end 172.9923 82.2428) (width 0.2) (layer "B.Cu") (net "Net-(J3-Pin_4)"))
 (segment (start 172.6051 81.8556) (end 172.6051 76.1022) (width 0.2) (layer "B.Cu") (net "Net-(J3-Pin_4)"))
 (segment (start 172.7569 82.0074) (end 172.6051 81.8556) (width 0.2) (layer "B.Cu") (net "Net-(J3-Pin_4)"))
 (segment (start 172.6051 76.1022) (end 172.4051 75.9022) (width 0.2) (layer "B.Cu") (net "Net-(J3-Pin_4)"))
 (segment (start 169 97.5) (end 169 96.3233) (width 0.2) (layer "B.Cu") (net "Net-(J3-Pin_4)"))
 (segment (start 172.9923 82.2428) (end 172.7569 82.0074) (width 0.2) (layer "B.Cu") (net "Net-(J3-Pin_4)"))
 (segment (start 172.7569 82.0074) (end 172.6051 81.8556) (width 0.2) (layer "B.Cu") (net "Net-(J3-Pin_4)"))
 (segment (start 172.189 75.7365) (end 172.189 73.7624) (width 0.2) (layer "B.Cu") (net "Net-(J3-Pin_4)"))
 (segment (start 172.4051 75.9022) (end 172.3547 75.9022) (width 0.2) (layer "B.Cu") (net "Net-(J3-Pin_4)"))
 (segment (start 170.5 71.3) (end 170.5 72.4017) (width 0.2) (layer "B.Cu") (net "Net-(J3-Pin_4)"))
 (segment (start 172.189 73.7624) (end 170.8283 72.4017) (width 0.2) (layer "B.Cu") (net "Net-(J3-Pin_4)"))
 (segment (start 170.8283 72.4017) (end 170.5 72.4017) (width 0.2) (layer "B.Cu") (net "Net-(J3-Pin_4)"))
 (segment (start 172.3547 75.9022) (end 172.189 75.7365) (width 0.2) (layer "B.Cu") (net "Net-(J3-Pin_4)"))
 (segment (start 169 96.3233) (end 169.3952 96.3233) (width 0.2) (layer "B.Cu") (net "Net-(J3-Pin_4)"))
 (segment (start 171.9017 97.5) (end 173.394 96.0077) (width 0.2) (layer "B.Cu") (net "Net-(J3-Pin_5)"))
 (segment (start 173.1586 81.8411) (end 173.0068 81.6893) (width 0.2) (layer "B.Cu") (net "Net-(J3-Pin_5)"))
 (segment (start 171 97.5) (end 171.9017 97.5) (width 0.2) (layer "B.Cu") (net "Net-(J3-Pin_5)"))
 (segment (start 172.2034 71.6747) (end 172.2034 71.152) (width 0.2) (layer "B.Cu") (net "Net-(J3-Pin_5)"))
 (segment (start 172.7714 75.7005) (end 172.6051 75.5342) (width 0.2) (layer "B.Cu") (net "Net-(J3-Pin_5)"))
 (segment (start 173.394 82.0765) (end 173.1586 81.8411) (width 0.2) (layer "B.Cu") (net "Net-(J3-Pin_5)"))
 (segment (start 172.6051 75.5342) (end 172.6051 72.0764) (width 0.2) (layer "B.Cu") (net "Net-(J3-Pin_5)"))
 (segment (start 173.1586 81.8411) (end 173.0068 81.6893) (width 0.2) (layer "B.Cu") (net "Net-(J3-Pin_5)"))
 (segment (start 170.9131 69.8617) (end 170.5 69.8617) (width 0.2) (layer "B.Cu") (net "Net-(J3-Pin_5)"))
 (segment (start 173.0068 75.9359) (end 172.7714 75.7005) (width 0.2) (layer "B.Cu") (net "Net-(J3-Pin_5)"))
 (segment (start 172.6051 72.0764) (end 172.2034 71.6747) (width 0.2) (layer "B.Cu") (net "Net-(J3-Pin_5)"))
 (segment (start 173.0068 81.6893) (end 173.0068 75.9359) (width 0.2) (layer "B.Cu") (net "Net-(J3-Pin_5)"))
 (segment (start 173.394 96.0077) (end 173.394 82.0765) (width 0.2) (layer "B.Cu") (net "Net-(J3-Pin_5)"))
 (segment (start 172.2034 71.152) (end 170.9131 69.8617) (width 0.2) (layer "B.Cu") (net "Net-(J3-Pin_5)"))
 (segment (start 172.7714 75.7005) (end 172.6051 75.5342) (width 0.2) (layer "B.Cu") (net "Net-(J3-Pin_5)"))
 (segment (start 170.5 68.76) (end 170.5 69.8617) (width 0.2) (layer "B.Cu") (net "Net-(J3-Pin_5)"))
 (segment (start 147.3117 74.9417) (end 145.0978 77.1556) (width 0.2) (layer "B.Cu") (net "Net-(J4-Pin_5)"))
 (segment (start 145.0978 77.1556) (end 145.0978 96.941) (width 0.2) (layer "B.Cu") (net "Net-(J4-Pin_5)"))
 (segment (start 155.0983 98.0636) (end 155.0983 97.5) (width 0.2) (layer "B.Cu") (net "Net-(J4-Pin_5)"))
 (segment (start 145.0978 96.941) (end 147.2365 99.0797) (width 0.2) (layer "B.Cu") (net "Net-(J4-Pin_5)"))
 (segment (start 154.0822 99.0797) (end 155.0983 98.0636) (width 0.2) (layer "B.Cu") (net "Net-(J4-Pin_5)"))
 (segment (start 147.64 73.84) (end 147.64 74.9417) (width 0.2) (layer "B.Cu") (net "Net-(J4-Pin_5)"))
 (segment (start 147.64 74.9417) (end 147.3117 74.9417) (width 0.2) (layer "B.Cu") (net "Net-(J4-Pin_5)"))
 (segment (start 156 97.5) (end 155.0983 97.5) (width 0.2) (layer "B.Cu") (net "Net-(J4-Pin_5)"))
 (segment (start 147.2365 99.0797) (end 154.0822 99.0797) (width 0.2) (layer "B.Cu") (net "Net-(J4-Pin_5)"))
 (segment (start 147.3117 77.4817) (end 147.64 77.4817) (width 0.2) (layer "B.Cu") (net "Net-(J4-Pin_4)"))
 (segment (start 153.0983 97.5) (end 153.0983 97.9565) (width 0.2) (layer "B.Cu") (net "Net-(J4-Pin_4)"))
 (segment (start 154 97.5) (end 153.0983 97.5) (width 0.2) (layer "B.Cu") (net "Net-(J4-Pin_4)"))
 (segment (start 147.4028 98.678) (end 146.8318 98.107) (width 0.2) (layer "B.Cu") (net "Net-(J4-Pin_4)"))
 (segment (start 153.0983 97.9565) (end 152.3768 98.678) (width 0.2) (layer "B.Cu") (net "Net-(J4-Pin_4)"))
 (segment (start 146.8318 98.107) (end 146.8318 93.989) (width 0.2) (layer "B.Cu") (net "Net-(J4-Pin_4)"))
 (segment (start 147.64 76.38) (end 147.64 77.4817) (width 0.2) (layer "B.Cu") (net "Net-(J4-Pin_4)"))
 (segment (start 152.3768 98.678) (end 147.4028 98.678) (width 0.2) (layer "B.Cu") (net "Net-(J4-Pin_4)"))
 (segment (start 145.4995 92.6567) (end 145.4995 79.2939) (width 0.2) (layer "B.Cu") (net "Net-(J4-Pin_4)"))
 (segment (start 145.4995 79.2939) (end 147.3117 77.4817) (width 0.2) (layer "B.Cu") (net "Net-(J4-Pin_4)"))
 (segment (start 146.8318 93.989) (end 145.4995 92.6567) (width 0.2) (layer "B.Cu") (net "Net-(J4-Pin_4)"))
 (segment (start 151.0983 97.0367) (end 147.1359 93.0743) (width 0.2) (layer "B.Cu") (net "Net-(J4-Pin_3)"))
 (segment (start 147.1359 93.0743) (end 146.6975 93.0743) (width 0.2) (layer "B.Cu") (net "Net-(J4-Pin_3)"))
 (segment (start 151.0983 97.5) (end 151.0983 97.0367) (width 0.2) (layer "B.Cu") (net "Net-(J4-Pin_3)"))
 (segment (start 145.9133 81.4201) (end 147.3117 80.0217) (width 0.2) (layer "B.Cu") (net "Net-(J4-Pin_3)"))
 (segment (start 152 97.5) (end 151.0983 97.5) (width 0.2) (layer "B.Cu") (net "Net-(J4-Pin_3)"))
 (segment (start 147.3117 80.0217) (end 147.64 80.0217) (width 0.2) (layer "B.Cu") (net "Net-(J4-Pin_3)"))
 (segment (start 145.9133 92.2901) (end 145.9133 81.4201) (width 0.2) (layer "B.Cu") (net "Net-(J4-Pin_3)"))
 (segment (start 147.64 78.92) (end 147.64 80.0217) (width 0.2) (layer "B.Cu") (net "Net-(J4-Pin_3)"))
 (segment (start 146.6975 93.0743) (end 145.9133 92.2901) (width 0.2) (layer "B.Cu") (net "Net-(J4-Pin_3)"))
 (segment (start 147.64 81.46) (end 144.1066 81.46) (width 0.2) (layer "F.Cu") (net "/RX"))
 (segment (start 144.1066 81.46) (end 143.7618 81.8048) (width 0.2) (layer "F.Cu") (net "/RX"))
 (via (at 143.7618 81.8048) (size 0.6) (drill 0.3) (layers "F.Cu" "B.Cu") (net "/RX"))
 (segment (start 143.7618 87.6982) (end 141.5 89.96) (width 0.2) (layer "B.Cu") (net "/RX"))
 (segment (start 143.7618 81.8048) (end 143.7618 87.6982) (width 0.2) (layer "B.Cu") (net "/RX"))
 (segment (start 142.6517 87.6866) (end 142.6517 90.4846) (width 0.2) (layer "F.Cu") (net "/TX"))
 (segment (start 141.788 91.3483) (end 141.5 91.3483) (width 0.2) (layer "F.Cu") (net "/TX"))
 (segment (start 146.3383 84) (end 142.6517 87.6866) (width 0.2) (layer "F.Cu") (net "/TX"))
 (segment (start 141.5 92.5) (end 141.5 91.3483) (width 0.2) (layer "F.Cu") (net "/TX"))
 (segment (start 142.6517 90.4846) (end 141.788 91.3483) (width 0.2) (layer "F.Cu") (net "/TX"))
 (segment (start 147.64 84) (end 146.3383 84) (width 0.2) (layer "F.Cu") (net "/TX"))
 (segment (start 124.2502 102.0042) (end 130.2102 102.0042) (width 0.2) (layer "F.Cu") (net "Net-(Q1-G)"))
 (segment (start 130.2102 102.0042) (end 130.2502 102.0442) (width 0.2) (layer "F.Cu") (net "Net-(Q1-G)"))
 (segment (start 119.2502 98.1384) (end 120.3844 98.1384) (width 0.2) (layer "B.Cu") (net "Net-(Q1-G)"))
 (segment (start 119.2502 96.8842) (end 119.2502 98.1384) (width 0.2) (layer "B.Cu") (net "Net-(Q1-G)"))
 (segment (start 120.3844 98.1384) (end 124.2502 102.0042) (width 0.2) (layer "B.Cu") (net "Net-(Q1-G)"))
 (segment (start 144.8442 94.3442) (end 148 97.5) (width 0.2) (layer "F.Cu") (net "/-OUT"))
 (segment (start 148 97.5) (end 149.1911 98.6911) (width 0.2) (layer "F.Cu") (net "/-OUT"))
 (segment (start 161.8089 98.6911) (end 163 97.5) (width 0.2) (layer "F.Cu") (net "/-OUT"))
 (segment (start 149.1911 98.6911) (end 161.8089 98.6911) (width 0.2) (layer "F.Cu") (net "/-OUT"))
 (segment (start 119.2502 94.3442) (end 144.8442 94.3442) (width 0.2) (layer "F.Cu") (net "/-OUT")))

